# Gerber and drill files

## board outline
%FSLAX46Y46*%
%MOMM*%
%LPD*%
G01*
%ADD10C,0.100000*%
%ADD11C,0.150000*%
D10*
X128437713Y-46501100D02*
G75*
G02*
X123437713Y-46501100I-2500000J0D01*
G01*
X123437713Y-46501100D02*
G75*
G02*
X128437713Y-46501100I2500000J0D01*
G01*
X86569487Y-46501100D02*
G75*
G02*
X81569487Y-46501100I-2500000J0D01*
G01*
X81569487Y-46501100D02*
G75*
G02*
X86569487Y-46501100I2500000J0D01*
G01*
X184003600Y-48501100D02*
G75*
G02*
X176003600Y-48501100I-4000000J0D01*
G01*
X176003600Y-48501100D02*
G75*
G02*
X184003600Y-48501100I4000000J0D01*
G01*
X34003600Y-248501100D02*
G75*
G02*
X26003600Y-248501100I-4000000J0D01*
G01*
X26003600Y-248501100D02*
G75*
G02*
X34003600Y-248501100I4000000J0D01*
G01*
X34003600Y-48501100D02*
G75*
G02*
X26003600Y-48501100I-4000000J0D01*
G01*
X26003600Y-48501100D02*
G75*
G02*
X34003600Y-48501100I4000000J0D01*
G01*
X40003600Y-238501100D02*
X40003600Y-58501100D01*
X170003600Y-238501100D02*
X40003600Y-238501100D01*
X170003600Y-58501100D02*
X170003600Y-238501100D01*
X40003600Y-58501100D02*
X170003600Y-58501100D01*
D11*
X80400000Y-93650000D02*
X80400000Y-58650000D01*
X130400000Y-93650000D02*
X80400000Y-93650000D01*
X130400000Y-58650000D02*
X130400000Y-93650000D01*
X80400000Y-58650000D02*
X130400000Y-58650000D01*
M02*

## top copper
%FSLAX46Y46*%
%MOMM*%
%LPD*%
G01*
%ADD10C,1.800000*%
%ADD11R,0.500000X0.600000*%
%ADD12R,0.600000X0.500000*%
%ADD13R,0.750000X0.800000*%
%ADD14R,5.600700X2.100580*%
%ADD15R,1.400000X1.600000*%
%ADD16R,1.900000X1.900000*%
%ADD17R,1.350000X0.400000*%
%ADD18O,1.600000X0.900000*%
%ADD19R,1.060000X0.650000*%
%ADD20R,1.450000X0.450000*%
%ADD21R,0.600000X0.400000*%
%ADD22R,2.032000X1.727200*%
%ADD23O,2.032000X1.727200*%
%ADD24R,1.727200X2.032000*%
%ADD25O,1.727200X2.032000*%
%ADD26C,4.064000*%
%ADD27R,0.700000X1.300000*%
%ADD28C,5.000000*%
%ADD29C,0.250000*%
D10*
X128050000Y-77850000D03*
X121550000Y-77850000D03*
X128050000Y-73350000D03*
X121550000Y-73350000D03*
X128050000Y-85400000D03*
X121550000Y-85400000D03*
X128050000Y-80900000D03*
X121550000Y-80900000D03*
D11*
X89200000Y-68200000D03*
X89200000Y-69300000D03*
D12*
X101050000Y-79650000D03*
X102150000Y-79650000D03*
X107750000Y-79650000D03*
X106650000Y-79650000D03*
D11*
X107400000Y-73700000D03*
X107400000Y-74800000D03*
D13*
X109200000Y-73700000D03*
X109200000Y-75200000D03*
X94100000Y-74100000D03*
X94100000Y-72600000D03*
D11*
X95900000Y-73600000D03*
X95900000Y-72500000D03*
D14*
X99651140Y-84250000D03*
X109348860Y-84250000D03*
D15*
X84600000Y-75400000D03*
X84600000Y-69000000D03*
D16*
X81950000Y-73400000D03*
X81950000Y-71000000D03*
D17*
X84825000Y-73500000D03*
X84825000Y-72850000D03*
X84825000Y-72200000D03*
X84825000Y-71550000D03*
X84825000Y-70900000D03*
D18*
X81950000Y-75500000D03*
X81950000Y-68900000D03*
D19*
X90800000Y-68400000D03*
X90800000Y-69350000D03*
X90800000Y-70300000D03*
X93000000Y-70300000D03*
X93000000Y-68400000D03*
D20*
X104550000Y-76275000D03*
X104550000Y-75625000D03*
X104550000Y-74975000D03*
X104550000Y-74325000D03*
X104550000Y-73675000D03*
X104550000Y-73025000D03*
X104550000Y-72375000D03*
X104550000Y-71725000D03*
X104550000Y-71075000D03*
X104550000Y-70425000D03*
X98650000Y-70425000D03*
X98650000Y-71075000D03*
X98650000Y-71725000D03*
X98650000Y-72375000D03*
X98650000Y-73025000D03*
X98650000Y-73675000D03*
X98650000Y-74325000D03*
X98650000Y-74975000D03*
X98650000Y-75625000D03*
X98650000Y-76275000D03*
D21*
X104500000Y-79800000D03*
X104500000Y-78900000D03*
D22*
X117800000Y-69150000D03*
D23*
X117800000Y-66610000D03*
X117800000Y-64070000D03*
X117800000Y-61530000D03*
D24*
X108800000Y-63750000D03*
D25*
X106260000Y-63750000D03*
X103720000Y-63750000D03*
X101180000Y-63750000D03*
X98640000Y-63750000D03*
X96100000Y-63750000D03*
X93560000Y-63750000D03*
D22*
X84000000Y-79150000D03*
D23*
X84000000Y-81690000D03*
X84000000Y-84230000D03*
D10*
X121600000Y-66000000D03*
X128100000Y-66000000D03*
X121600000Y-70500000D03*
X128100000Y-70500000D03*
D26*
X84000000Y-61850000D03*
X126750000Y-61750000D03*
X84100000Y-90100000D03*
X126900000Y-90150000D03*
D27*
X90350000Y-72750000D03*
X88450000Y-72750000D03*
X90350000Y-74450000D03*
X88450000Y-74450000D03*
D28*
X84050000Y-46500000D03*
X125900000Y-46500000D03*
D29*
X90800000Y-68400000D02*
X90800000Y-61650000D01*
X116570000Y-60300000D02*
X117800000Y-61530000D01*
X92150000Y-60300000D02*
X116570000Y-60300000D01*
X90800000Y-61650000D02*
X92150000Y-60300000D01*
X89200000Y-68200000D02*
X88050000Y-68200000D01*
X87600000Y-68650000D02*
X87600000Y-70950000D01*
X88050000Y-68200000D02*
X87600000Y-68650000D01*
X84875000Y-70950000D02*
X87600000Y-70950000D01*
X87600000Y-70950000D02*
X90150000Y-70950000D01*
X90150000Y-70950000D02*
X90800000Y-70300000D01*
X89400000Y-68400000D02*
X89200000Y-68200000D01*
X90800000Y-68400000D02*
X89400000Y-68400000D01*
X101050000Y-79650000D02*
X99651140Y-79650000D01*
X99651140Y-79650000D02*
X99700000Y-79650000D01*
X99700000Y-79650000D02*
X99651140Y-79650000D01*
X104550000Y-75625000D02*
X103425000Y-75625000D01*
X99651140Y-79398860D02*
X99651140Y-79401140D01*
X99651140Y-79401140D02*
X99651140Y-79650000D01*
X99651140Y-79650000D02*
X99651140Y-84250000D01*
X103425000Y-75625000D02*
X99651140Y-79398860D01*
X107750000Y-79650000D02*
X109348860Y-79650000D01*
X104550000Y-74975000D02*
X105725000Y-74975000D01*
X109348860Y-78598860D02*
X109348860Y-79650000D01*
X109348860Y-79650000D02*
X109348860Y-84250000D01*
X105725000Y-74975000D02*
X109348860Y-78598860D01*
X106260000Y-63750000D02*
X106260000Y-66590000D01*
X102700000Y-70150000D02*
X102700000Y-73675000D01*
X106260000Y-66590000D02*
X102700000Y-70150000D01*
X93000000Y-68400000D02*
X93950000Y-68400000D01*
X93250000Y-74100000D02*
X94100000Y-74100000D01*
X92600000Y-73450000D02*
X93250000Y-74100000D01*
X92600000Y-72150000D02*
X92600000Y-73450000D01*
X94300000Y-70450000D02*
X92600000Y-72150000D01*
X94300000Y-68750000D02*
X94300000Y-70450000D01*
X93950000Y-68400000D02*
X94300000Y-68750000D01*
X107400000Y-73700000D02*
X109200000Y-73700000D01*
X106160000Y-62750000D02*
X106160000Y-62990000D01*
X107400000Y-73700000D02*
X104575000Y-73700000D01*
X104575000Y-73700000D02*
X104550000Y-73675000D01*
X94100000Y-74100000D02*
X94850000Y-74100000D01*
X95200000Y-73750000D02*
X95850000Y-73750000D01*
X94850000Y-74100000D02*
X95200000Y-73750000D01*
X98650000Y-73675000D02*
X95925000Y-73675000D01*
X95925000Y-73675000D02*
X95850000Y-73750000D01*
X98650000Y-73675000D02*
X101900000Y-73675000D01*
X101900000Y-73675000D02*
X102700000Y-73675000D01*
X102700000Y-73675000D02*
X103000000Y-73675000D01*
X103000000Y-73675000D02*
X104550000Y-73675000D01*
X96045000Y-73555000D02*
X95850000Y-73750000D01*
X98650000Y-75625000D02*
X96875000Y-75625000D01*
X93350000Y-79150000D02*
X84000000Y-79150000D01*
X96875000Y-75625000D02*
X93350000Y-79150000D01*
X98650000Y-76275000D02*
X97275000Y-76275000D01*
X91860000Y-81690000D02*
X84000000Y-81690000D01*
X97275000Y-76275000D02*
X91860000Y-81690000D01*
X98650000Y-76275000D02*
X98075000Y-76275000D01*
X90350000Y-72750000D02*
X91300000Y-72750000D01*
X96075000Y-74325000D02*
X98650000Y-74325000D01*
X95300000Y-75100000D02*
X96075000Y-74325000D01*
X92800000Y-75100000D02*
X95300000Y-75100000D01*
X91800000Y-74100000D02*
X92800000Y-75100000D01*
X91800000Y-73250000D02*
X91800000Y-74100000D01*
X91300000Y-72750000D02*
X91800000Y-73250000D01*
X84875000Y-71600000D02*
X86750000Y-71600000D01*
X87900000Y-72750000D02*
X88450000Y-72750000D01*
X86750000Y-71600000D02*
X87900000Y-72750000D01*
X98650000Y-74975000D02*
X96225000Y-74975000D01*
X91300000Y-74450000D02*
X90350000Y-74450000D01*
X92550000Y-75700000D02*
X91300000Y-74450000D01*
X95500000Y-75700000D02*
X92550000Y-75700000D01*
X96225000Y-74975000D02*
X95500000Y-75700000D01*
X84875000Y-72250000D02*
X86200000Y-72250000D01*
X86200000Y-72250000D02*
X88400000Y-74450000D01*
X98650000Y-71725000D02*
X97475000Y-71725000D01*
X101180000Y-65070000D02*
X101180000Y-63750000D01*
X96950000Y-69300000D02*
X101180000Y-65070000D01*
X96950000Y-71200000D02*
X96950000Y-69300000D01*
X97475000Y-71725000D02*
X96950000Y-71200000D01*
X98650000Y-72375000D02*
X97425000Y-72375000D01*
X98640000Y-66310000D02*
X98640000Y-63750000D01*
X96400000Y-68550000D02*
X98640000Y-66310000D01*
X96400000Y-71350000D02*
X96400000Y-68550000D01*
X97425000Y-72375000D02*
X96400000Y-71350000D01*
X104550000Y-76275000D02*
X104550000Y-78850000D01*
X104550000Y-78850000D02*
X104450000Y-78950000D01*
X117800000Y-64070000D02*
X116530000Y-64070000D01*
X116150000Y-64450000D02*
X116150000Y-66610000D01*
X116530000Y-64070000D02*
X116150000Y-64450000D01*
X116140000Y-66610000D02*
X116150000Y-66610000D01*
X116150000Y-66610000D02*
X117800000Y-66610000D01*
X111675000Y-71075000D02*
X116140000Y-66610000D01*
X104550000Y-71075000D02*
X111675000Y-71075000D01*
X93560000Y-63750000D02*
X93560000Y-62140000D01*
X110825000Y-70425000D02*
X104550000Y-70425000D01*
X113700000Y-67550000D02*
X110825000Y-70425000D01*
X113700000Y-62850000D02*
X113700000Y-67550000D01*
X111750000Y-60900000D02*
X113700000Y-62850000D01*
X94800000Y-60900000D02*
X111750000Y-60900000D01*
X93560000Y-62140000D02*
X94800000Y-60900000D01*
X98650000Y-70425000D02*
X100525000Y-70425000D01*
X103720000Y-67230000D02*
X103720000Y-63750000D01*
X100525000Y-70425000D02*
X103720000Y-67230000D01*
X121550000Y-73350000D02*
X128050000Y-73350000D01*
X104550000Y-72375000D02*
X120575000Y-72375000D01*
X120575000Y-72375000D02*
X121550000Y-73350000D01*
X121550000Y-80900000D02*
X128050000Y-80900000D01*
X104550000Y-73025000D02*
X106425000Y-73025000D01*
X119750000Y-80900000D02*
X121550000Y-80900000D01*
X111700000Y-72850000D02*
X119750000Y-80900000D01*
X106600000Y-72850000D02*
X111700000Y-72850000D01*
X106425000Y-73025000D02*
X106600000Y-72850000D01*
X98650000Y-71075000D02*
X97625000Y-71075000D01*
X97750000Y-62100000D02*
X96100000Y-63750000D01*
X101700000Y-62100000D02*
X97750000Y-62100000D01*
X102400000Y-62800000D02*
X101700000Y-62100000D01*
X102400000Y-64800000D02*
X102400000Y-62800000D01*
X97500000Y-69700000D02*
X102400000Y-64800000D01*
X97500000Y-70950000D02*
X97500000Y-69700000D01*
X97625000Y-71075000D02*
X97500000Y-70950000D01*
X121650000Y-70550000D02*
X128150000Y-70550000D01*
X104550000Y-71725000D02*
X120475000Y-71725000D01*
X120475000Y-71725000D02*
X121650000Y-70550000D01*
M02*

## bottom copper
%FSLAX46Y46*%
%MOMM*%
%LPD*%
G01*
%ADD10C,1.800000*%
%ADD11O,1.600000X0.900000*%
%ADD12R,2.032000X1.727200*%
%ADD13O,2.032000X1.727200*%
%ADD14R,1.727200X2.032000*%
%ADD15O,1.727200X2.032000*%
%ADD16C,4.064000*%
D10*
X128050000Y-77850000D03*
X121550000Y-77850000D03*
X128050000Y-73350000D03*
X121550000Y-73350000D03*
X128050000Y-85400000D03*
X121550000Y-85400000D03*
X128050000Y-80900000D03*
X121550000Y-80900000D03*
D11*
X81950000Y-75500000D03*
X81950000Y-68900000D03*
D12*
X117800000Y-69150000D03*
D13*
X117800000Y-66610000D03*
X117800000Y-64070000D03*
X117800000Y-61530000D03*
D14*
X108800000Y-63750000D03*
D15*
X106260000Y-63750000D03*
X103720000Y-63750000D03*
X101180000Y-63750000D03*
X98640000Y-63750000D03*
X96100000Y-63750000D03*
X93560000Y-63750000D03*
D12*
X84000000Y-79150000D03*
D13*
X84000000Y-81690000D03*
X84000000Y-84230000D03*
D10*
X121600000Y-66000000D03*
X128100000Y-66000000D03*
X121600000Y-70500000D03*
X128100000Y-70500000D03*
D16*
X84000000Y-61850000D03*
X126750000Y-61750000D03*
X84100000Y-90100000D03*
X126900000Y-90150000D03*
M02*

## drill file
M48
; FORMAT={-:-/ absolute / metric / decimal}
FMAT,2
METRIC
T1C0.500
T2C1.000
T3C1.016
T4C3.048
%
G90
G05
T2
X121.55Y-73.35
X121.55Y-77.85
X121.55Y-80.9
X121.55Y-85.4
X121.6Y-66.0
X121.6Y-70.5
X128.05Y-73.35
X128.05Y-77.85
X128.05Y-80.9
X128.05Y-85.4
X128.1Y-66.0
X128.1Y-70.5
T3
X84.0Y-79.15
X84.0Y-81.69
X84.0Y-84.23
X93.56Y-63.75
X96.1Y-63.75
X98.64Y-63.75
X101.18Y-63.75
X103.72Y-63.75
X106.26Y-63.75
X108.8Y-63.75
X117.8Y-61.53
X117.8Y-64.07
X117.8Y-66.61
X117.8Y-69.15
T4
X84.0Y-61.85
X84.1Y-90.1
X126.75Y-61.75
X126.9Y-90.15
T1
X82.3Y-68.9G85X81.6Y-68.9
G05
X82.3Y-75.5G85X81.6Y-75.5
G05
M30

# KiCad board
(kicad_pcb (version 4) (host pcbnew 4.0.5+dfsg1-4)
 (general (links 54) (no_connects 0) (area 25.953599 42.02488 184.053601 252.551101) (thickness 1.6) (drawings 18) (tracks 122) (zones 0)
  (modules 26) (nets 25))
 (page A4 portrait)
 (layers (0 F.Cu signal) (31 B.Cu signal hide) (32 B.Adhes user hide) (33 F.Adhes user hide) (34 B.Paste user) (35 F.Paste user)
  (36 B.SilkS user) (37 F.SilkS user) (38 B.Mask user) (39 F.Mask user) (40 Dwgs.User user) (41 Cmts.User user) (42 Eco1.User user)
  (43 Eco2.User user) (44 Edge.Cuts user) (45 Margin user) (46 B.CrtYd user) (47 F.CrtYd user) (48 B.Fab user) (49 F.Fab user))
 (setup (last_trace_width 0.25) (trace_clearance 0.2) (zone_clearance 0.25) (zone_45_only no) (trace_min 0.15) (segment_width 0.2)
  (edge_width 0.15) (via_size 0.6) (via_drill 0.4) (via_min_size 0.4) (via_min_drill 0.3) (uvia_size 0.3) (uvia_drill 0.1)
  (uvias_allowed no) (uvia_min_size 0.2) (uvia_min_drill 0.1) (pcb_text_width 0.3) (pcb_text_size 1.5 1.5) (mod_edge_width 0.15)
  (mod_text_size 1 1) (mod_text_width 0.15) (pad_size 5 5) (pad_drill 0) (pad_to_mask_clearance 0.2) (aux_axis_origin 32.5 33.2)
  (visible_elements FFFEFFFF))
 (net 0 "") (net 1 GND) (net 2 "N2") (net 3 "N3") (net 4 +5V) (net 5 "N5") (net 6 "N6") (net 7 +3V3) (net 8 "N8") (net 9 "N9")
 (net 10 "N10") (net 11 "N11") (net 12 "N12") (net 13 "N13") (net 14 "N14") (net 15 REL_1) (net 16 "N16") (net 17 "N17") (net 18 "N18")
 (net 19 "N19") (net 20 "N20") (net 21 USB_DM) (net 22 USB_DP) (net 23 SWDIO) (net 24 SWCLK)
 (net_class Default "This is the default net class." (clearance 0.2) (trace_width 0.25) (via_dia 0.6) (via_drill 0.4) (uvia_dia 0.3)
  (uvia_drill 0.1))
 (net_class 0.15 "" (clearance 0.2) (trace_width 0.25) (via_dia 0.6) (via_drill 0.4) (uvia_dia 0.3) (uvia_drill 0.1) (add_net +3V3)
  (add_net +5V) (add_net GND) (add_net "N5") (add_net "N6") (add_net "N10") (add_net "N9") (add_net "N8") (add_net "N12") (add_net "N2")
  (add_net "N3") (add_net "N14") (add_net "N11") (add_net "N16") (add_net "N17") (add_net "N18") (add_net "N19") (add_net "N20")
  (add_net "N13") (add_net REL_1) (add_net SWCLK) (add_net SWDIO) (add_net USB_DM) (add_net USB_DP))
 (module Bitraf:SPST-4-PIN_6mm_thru (layer B.Cu) (at 124.8 75.6 180)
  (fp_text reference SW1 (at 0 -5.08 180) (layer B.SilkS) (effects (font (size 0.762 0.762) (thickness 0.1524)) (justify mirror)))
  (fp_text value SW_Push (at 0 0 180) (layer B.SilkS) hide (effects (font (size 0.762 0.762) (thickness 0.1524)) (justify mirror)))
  (pad 1 thru_hole circle (at -3.25 -2.25 180) (size 1.8 1.8) (drill 1) (layers *.Cu *.Mask B.SilkS) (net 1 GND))
  (pad 1 thru_hole circle (at 3.25 -2.25 180) (size 1.8 1.8) (drill 1) (layers *.Cu *.Mask B.SilkS) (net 1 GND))
  (pad 2 thru_hole circle (at -3.25 2.25 180) (size 1.8 1.8) (drill 1) (layers *.Cu *.Mask B.SilkS) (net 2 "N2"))
  (pad 2 thru_hole circle (at 3.25 2.25 180) (size 1.8 1.8) (drill 1) (layers *.Cu *.Mask B.SilkS) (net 2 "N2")))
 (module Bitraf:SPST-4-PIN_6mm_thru (layer B.Cu) (at 124.8 83.15 180)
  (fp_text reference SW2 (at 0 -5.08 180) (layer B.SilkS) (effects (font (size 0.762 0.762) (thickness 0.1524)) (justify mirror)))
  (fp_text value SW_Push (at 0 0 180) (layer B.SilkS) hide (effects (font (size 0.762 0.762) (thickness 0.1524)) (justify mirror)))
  (pad 1 thru_hole circle (at -3.25 -2.25 180) (size 1.8 1.8) (drill 1) (layers *.Cu *.Mask B.SilkS) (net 1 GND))
  (pad 1 thru_hole circle (at 3.25 -2.25 180) (size 1.8 1.8) (drill 1) (layers *.Cu *.Mask B.SilkS) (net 1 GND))
  (pad 2 thru_hole circle (at -3.25 2.25 180) (size 1.8 1.8) (drill 1) (layers *.Cu *.Mask B.SilkS) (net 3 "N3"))
  (pad 2 thru_hole circle (at 3.25 2.25 180) (size 1.8 1.8) (drill 1) (layers *.Cu *.Mask B.SilkS) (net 3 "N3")))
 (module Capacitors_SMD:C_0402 (layer F.Cu) (at 89.2 68.75 270)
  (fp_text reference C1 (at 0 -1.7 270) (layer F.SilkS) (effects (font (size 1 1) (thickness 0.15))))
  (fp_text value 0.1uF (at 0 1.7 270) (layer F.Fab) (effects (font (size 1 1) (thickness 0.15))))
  (pad 1 smd rect (at -0.55 0 270) (size 0.6 0.5) (layers F.Cu F.Paste F.Mask) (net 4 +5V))
  (pad 2 smd rect (at 0.55 0 270) (size 0.6 0.5) (layers F.Cu F.Paste F.Mask) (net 1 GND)))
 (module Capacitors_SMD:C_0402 (layer F.Cu) (at 101.6 79.65)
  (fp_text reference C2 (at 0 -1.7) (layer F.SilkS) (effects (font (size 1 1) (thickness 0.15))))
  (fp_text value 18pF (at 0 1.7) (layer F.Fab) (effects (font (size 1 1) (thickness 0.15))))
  (pad 1 smd rect (at -0.55 0) (size 0.6 0.5) (layers F.Cu F.Paste F.Mask) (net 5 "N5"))
  (pad 2 smd rect (at 0.55 0) (size 0.6 0.5) (layers F.Cu F.Paste F.Mask) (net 1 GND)))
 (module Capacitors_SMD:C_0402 (layer F.Cu) (at 107.2 79.65 180)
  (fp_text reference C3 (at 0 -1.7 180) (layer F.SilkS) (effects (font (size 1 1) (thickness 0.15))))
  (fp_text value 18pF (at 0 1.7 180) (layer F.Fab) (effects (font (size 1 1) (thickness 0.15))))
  (pad 1 smd rect (at -0.55 0 180) (size 0.6 0.5) (layers F.Cu F.Paste F.Mask) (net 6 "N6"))
  (pad 2 smd rect (at 0.55 0 180) (size 0.6 0.5) (layers F.Cu F.Paste F.Mask) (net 1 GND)))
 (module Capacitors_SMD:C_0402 (layer F.Cu) (at 107.4 74.25 270)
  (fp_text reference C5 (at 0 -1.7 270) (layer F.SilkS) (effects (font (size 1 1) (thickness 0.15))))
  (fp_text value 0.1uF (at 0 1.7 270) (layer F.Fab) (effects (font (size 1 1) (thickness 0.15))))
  (pad 1 smd rect (at -0.55 0 270) (size 0.6 0.5) (layers F.Cu F.Paste F.Mask) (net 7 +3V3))
  (pad 2 smd rect (at 0.55 0 270) (size 0.6 0.5) (layers F.Cu F.Paste F.Mask) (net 1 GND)))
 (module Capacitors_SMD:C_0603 (layer F.Cu) (at 109.2 74.45 270)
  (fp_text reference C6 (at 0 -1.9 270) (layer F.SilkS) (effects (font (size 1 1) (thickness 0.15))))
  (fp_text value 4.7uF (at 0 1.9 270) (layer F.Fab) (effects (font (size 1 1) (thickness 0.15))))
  (pad 1 smd rect (at -0.75 0 270) (size 0.8 0.75) (layers F.Cu F.Paste F.Mask) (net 7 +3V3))
  (pad 2 smd rect (at 0.75 0 270) (size 0.8 0.75) (layers F.Cu F.Paste F.Mask) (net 1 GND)))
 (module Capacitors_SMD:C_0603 (layer F.Cu) (at 94.1 73.35 90)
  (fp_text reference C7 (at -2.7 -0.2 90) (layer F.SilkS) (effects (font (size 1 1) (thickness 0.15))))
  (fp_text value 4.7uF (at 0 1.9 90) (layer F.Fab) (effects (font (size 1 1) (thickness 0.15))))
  (pad 1 smd rect (at -0.75 0 90) (size 0.8 0.75) (layers F.Cu F.Paste F.Mask) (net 7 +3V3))
  (pad 2 smd rect (at 0.75 0 90) (size 0.8 0.75) (layers F.Cu F.Paste F.Mask) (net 1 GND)))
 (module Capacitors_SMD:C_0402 (layer F.Cu) (at 95.9 73.05 90)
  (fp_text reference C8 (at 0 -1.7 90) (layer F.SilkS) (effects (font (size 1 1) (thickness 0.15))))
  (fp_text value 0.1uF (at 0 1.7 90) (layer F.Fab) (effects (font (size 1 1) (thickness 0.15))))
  (pad 1 smd rect (at -0.55 0 90) (size 0.6 0.5) (layers F.Cu F.Paste F.Mask) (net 7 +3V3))
  (pad 2 smd rect (at 0.55 0 90) (size 0.6 0.5) (layers F.Cu F.Paste F.Mask) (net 1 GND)))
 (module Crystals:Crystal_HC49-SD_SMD (layer F.Cu) (at 104.5 84.25)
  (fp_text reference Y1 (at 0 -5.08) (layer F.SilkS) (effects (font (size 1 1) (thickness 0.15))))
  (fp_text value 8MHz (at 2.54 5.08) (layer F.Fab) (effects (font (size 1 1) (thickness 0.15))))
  (pad 1 smd rect (at -4.84886 0) (size 5.6007 2.10058) (layers F.Cu F.Paste F.Mask) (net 5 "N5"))
  (pad 2 smd rect (at 4.84886 0) (size 5.6007 2.10058) (layers F.Cu F.Paste F.Mask) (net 6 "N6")))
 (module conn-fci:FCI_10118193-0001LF (layer F.Cu) (at 81.95 72.2 270) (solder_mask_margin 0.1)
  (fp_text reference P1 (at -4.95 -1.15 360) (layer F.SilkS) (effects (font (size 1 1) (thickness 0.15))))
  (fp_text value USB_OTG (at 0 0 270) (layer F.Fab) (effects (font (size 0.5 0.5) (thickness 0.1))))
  (pad SH smd rect (at 3.2 -2.65 270) (size 1.6 1.4) (layers F.Cu F.Paste F.Mask))
  (pad SH smd rect (at -3.2 -2.65 270) (size 1.6 1.4) (layers F.Cu F.Paste F.Mask))
  (pad SH smd rect (at 1.2 0 270) (size 1.9 1.9) (layers F.Cu F.Paste F.Mask))
  (pad SH smd rect (at -1.2 0 270) (size 1.9 1.9) (layers F.Cu F.Paste F.Mask))
  (pad 5 smd rect (at 1.3 -2.875 270) (size 0.4 1.35) (layers F.Cu F.Paste F.Mask) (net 1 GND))
  (pad 4 smd rect (at 0.65 -2.875 270) (size 0.4 1.35) (layers F.Cu F.Paste F.Mask) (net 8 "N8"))
  (pad 3 smd rect (at 0 -2.875 270) (size 0.4 1.35) (layers F.Cu F.Paste F.Mask) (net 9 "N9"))
  (pad 2 smd rect (at -0.65 -2.875 270) (size 0.4 1.35) (layers F.Cu F.Paste F.Mask) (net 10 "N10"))
  (pad 1 smd rect (at -1.3 -2.875 270) (size 0.4 1.35) (layers F.Cu F.Paste F.Mask) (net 4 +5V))
  (pad SH thru_hole oval (at 3.3 0 270) (size 0.9 1.6) (drill oval 0.5 1.2) (layers *.Cu *.Mask))
  (pad SH thru_hole oval (at -3.3 0 270) (size 0.9 1.6) (drill oval 0.5 1.2) (layers *.Cu *.Mask)))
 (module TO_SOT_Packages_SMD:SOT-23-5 (layer F.Cu) (at 91.9 69.35)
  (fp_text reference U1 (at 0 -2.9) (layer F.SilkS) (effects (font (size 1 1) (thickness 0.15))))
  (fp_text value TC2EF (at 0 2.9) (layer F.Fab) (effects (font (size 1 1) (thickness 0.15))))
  (pad 1 smd rect (at -1.1 -0.95) (size 1.06 0.65) (layers F.Cu F.Paste F.Mask) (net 4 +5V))
  (pad 2 smd rect (at -1.1 0) (size 1.06 0.65) (layers F.Cu F.Paste F.Mask) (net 1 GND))
  (pad 3 smd rect (at -1.1 0.95) (size 1.06 0.65) (layers F.Cu F.Paste F.Mask) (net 4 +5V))
  (pad 4 smd rect (at 1.1 0.95) (size 1.06 0.65) (layers F.Cu F.Paste F.Mask) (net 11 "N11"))
  (pad 5 smd rect (at 1.1 -0.95) (size 1.06 0.65) (layers F.Cu F.Paste F.Mask) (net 7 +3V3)))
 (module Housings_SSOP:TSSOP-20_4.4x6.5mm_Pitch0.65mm (layer F.Cu) (at 101.6 73.35 180)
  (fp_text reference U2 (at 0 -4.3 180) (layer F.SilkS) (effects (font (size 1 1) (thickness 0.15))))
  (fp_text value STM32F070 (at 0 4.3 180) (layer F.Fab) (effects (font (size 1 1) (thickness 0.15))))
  (pad 1 smd rect (at -2.95 -2.925 180) (size 1.45 0.45) (layers F.Cu F.Paste F.Mask) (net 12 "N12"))
  (pad 2 smd rect (at -2.95 -2.275 180) (size 1.45 0.45) (layers F.Cu F.Paste F.Mask) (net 5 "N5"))
  (pad 3 smd rect (at -2.95 -1.625 180) (size 1.45 0.45) (layers F.Cu F.Paste F.Mask) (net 6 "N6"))
  (pad 4 smd rect (at -2.95 -0.975 180) (size 1.45 0.45) (layers F.Cu F.Paste F.Mask) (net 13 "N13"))
  (pad 5 smd rect (at -2.95 -0.325 180) (size 1.45 0.45) (layers F.Cu F.Paste F.Mask) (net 7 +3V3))
  (pad 6 smd rect (at -2.95 0.325 180) (size 1.45 0.45) (layers F.Cu F.Paste F.Mask) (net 3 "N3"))
  (pad 7 smd rect (at -2.95 0.975 180) (size 1.45 0.45) (layers F.Cu F.Paste F.Mask) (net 2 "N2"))
  (pad 8 smd rect (at -2.95 1.625 180) (size 1.45 0.45) (layers F.Cu F.Paste F.Mask) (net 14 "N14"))
  (pad 9 smd rect (at -2.95 2.275 180) (size 1.45 0.45) (layers F.Cu F.Paste F.Mask) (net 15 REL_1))
  (pad 10 smd rect (at -2.95 2.925 180) (size 1.45 0.45) (layers F.Cu F.Paste F.Mask) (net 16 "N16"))
  (pad 11 smd rect (at 2.95 2.925 180) (size 1.45 0.45) (layers F.Cu F.Paste F.Mask) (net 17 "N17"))
  (pad 12 smd rect (at 2.95 2.275 180) (size 1.45 0.45) (layers F.Cu F.Paste F.Mask) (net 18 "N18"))
  (pad 13 smd rect (at 2.95 1.625 180) (size 1.45 0.45) (layers F.Cu F.Paste F.Mask) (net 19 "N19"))
  (pad 14 smd rect (at 2.95 0.975 180) (size 1.45 0.45) (layers F.Cu F.Paste F.Mask) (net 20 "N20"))
  (pad 15 smd rect (at 2.95 0.325 180) (size 1.45 0.45) (layers F.Cu F.Paste F.Mask) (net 1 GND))
  (pad 16 smd rect (at 2.95 -0.325 180) (size 1.45 0.45) (layers F.Cu F.Paste F.Mask) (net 7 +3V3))
  (pad 17 smd rect (at 2.95 -0.975 180) (size 1.45 0.45) (layers F.Cu F.Paste F.Mask) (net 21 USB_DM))
  (pad 18 smd rect (at 2.95 -1.625 180) (size 1.45 0.45) (layers F.Cu F.Paste F.Mask) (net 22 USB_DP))
  (pad 19 smd rect (at 2.95 -2.275 180) (size 1.45 0.45) (layers F.Cu F.Paste F.Mask) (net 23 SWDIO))
  (pad 20 smd rect (at 2.95 -2.925 180) (size 1.45 0.45) (layers F.Cu F.Paste F.Mask) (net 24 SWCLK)))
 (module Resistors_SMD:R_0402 (layer F.Cu) (at 104.5 79.35 90)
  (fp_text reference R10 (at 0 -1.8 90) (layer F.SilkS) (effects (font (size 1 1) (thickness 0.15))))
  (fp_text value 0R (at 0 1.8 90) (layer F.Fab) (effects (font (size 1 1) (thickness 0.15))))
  (pad 1 smd rect (at -0.45 0 90) (size 0.4 0.6) (layers F.Cu F.Paste F.Mask) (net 1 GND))
  (pad 2 smd rect (at 0.45 0 90) (size 0.4 0.6) (layers F.Cu F.Paste F.Mask) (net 12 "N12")))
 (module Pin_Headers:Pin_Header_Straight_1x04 (layer F.Cu) (at 117.8 69.15 180)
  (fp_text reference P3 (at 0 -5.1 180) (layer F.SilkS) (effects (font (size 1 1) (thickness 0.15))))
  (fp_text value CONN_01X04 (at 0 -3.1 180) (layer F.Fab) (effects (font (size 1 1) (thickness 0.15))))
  (pad 1 thru_hole rect (at 0 0 180) (size 2.032 1.7272) (drill 1.016) (layers *.Cu *.Mask) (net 1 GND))
  (pad 2 thru_hole oval (at 0 2.54 180) (size 2.032 1.7272) (drill 1.016) (layers *.Cu *.Mask) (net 15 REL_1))
  (pad 3 thru_hole oval (at 0 5.08 180) (size 2.032 1.7272) (drill 1.016) (layers *.Cu *.Mask) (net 15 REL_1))
  (pad 4 thru_hole oval (at 0 7.62 180) (size 2.032 1.7272) (drill 1.016) (layers *.Cu *.Mask) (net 4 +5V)))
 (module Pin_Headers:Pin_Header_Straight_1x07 (layer F.Cu) (at 108.8 63.75 270)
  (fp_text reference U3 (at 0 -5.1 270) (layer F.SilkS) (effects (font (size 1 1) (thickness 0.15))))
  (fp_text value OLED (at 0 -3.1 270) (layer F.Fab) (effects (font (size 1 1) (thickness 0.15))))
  (pad 1 thru_hole rect (at 0 0 270) (size 2.032 1.7272) (drill 1.016) (layers *.Cu *.Mask) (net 1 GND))
  (pad 2 thru_hole oval (at 0 2.54 270) (size 2.032 1.7272) (drill 1.016) (layers *.Cu *.Mask) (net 7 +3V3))
  (pad 3 thru_hole oval (at 0 5.08 270) (size 2.032 1.7272) (drill 1.016) (layers *.Cu *.Mask) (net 17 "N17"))
  (pad 4 thru_hole oval (at 0 7.62 270) (size 2.032 1.7272) (drill 1.016) (layers *.Cu *.Mask) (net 19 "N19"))
  (pad 5 thru_hole oval (at 0 10.16 270) (size 2.032 1.7272) (drill 1.016) (layers *.Cu *.Mask) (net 20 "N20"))
  (pad 6 thru_hole oval (at 0 12.7 270) (size 2.032 1.7272) (drill 1.016) (layers *.Cu *.Mask) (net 18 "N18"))
  (pad 7 thru_hole oval (at 0 15.24 270) (size 2.032 1.7272) (drill 1.016) (layers *.Cu *.Mask) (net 16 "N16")))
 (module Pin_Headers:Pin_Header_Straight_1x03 (layer F.Cu) (at 84 79.15)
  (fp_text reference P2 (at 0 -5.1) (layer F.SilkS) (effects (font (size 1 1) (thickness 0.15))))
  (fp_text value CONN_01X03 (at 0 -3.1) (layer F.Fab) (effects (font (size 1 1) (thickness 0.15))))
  (pad 1 thru_hole rect (at 0 0) (size 2.032 1.7272) (drill 1.016) (layers *.Cu *.Mask) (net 23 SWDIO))
  (pad 2 thru_hole oval (at 0 2.54) (size 2.032 1.7272) (drill 1.016) (layers *.Cu *.Mask) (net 24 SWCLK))
  (pad 3 thru_hole oval (at 0 5.08) (size 2.032 1.7272) (drill 1.016) (layers *.Cu *.Mask) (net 1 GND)))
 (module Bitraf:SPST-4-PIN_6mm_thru (layer B.Cu) (at 124.85 68.25)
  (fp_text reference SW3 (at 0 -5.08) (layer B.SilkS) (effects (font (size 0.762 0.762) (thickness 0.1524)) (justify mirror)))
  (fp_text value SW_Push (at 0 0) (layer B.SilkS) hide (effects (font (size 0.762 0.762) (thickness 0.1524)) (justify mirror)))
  (pad 1 thru_hole circle (at -3.25 -2.25) (size 1.8 1.8) (drill 1) (layers *.Cu *.Mask B.SilkS) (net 1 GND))
  (pad 1 thru_hole circle (at 3.25 -2.25) (size 1.8 1.8) (drill 1) (layers *.Cu *.Mask B.SilkS) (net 1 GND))
  (pad 2 thru_hole circle (at -3.25 2.25) (size 1.8 1.8) (drill 1) (layers *.Cu *.Mask B.SilkS) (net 14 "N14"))
  (pad 2 thru_hole circle (at 3.25 2.25) (size 1.8 1.8) (drill 1) (layers *.Cu *.Mask B.SilkS) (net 14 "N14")))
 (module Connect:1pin (layer F.Cu) (at 84 61.85)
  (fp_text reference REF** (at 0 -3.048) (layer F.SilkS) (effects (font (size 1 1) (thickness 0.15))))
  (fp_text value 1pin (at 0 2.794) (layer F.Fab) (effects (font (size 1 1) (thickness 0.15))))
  (pad 1 thru_hole circle (at 0 0) (size 4.064 4.064) (drill 3.048) (layers *.Cu *.Mask)))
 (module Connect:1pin (layer F.Cu) (at 126.75 61.75)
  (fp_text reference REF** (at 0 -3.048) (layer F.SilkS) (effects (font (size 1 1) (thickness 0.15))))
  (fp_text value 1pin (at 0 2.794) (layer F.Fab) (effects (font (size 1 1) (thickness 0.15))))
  (pad 1 thru_hole circle (at 0 0) (size 4.064 4.064) (drill 3.048) (layers *.Cu *.Mask)))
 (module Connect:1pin (layer F.Cu) (at 84.1 90.1)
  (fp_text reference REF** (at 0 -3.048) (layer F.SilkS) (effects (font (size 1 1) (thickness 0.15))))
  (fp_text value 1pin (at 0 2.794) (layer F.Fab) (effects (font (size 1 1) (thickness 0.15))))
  (pad 1 thru_hole circle (at 0 0) (size 4.064 4.064) (drill 3.048) (layers *.Cu *.Mask)))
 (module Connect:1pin (layer F.Cu) (at 126.9 90.15)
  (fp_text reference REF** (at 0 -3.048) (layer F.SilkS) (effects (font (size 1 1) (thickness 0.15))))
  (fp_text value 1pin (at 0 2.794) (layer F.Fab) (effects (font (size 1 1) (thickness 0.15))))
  (pad 1 thru_hole circle (at 0 0) (size 4.064 4.064) (drill 3.048) (layers *.Cu *.Mask)))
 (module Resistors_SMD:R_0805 (layer F.Cu) (at 89.4 72.75 180)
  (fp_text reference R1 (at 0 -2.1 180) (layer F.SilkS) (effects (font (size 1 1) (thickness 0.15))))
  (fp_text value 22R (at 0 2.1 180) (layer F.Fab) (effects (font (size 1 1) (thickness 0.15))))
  (pad 1 smd rect (at -0.95 0 180) (size 0.7 1.3) (layers F.Cu F.Paste F.Mask) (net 21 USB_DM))
  (pad 2 smd rect (at 0.95 0 180) (size 0.7 1.3) (layers F.Cu F.Paste F.Mask) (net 10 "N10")))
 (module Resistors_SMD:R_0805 (layer F.Cu) (at 89.4 74.45 180)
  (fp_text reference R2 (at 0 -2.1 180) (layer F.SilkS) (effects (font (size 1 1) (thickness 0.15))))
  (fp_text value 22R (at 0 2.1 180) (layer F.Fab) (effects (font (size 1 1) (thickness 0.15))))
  (pad 1 smd rect (at -0.95 0 180) (size 0.7 1.3) (layers F.Cu F.Paste F.Mask) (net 22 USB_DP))
  (pad 2 smd rect (at 0.95 0 180) (size 0.7 1.3) (layers F.Cu F.Paste F.Mask) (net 9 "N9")))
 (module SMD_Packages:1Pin (layer F.Cu) (at 84.05 46.5)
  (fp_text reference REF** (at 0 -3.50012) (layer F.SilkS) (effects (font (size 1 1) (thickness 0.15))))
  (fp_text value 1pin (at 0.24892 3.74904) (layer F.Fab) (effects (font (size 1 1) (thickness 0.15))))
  (pad 1 smd circle (at 0 0) (size 5 5) (layers F.Cu F.Paste F.Mask)))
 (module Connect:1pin (layer F.Cu) (at 125.9 46.5)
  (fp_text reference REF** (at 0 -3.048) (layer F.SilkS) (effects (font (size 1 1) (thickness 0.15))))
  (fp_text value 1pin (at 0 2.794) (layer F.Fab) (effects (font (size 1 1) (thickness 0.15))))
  (pad 1 smd circle (at 0 0) (size 5 5) (layers F.Cu F.Paste F.Mask)))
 (gr_circle (center 125.937713 46.5011) (end 128.437713 46.5011) (layer Edge.Cuts) (width 0.1))
 (gr_circle (center 84.069487 46.5011) (end 86.569487 46.5011) (layer Edge.Cuts) (width 0.1))
 (gr_circle (center 180.0036 48.5011) (end 184.0036 48.5011) (layer Edge.Cuts) (width 0.1))
 (gr_circle (center 30.0036 248.5011) (end 34.0036 248.5011) (layer Edge.Cuts) (width 0.1))
 (gr_circle (center 30.0036 48.5011) (end 34.0036 48.5011) (layer Edge.Cuts) (width 0.1))
 (gr_line (start 40.0036 238.5011) (end 40.0036 58.5011) (layer Edge.Cuts) (width 0.1))
 (gr_line (start 170.0036 238.5011) (end 40.0036 238.5011) (layer Edge.Cuts) (width 0.1))
 (gr_line (start 170.0036 58.5011) (end 170.0036 238.5011) (layer Edge.Cuts) (width 0.1))
 (gr_line (start 40.0036 58.5011) (end 170.0036 58.5011) (layer Edge.Cuts) (width 0.1))
 (gr_line (start 80.4 93.65) (end 80.4 58.65) (angle 90) (layer Edge.Cuts) (width 0.15))
 (gr_line (start 130.4 93.65) (end 80.4 93.65) (angle 90) (layer Edge.Cuts) (width 0.15))
 (gr_line (start 130.4 58.65) (end 130.4 93.65) (angle 90) (layer Edge.Cuts) (width 0.15))
 (gr_line (start 80.4 58.65) (end 130.4 58.65) (angle 90) (layer Edge.Cuts) (width 0.15))
 (segment (start 90.8 68.4) (end 90.8 61.65) (width 0.25) (layer F.Cu) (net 4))
 (segment (start 116.57 60.3) (end 117.8 61.53) (width 0.25) (layer F.Cu) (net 4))
 (segment (start 92.15 60.3) (end 116.57 60.3) (width 0.25) (layer F.Cu) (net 4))
 (segment (start 90.8 61.65) (end 92.15 60.3) (width 0.25) (layer F.Cu) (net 4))
 (segment (start 89.2 68.2) (end 88.05 68.2) (width 0.25) (layer F.Cu) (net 4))
 (segment (start 87.6 68.65) (end 87.6 70.95) (width 0.25) (layer F.Cu) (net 4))
 (segment (start 88.05 68.2) (end 87.6 68.65) (width 0.25) (layer F.Cu) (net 4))
 (segment (start 84.875 70.95) (end 87.6 70.95) (width 0.25) (layer F.Cu) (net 4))
 (segment (start 87.6 70.95) (end 90.15 70.95) (width 0.25) (layer F.Cu) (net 4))
 (segment (start 90.15 70.95) (end 90.8 70.3) (width 0.25) (layer F.Cu) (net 4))
 (segment (start 89.4 68.4) (end 89.2 68.2) (width 0.25) (layer F.Cu) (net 4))
 (segment (start 90.8 68.4) (end 89.4 68.4) (width 0.25) (layer F.Cu) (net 4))
 (segment (start 101.05 79.65) (end 99.65114 79.65) (width 0.25) (layer F.Cu) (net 5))
 (segment (start 99.65114 79.65) (end 99.7 79.65) (width 0.25) (layer F.Cu) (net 5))
 (segment (start 99.7 79.65) (end 99.65114 79.65) (width 0.25) (layer F.Cu) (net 5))
 (segment (start 104.55 75.625) (end 103.425 75.625) (width 0.25) (layer F.Cu) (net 5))
 (segment (start 99.65114 79.39886) (end 99.65114 79.40114) (width 0.25) (layer F.Cu) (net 5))
 (segment (start 99.65114 79.40114) (end 99.65114 79.65) (width 0.25) (layer F.Cu) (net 5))
 (segment (start 99.65114 79.65) (end 99.65114 84.25) (width 0.25) (layer F.Cu) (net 5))
 (segment (start 103.425 75.625) (end 99.65114 79.39886) (width 0.25) (layer F.Cu) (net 5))
 (segment (start 107.75 79.65) (end 109.34886 79.65) (width 0.25) (layer F.Cu) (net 6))
 (segment (start 104.55 74.975) (end 105.725 74.975) (width 0.25) (layer F.Cu) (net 6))
 (segment (start 109.34886 78.59886) (end 109.34886 79.65) (width 0.25) (layer F.Cu) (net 6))
 (segment (start 109.34886 79.65) (end 109.34886 84.25) (width 0.25) (layer F.Cu) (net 6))
 (segment (start 105.725 74.975) (end 109.34886 78.59886) (width 0.25) (layer F.Cu) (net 6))
 (segment (start 106.26 63.75) (end 106.26 66.59) (width 0.25) (layer F.Cu) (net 7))
 (segment (start 102.7 70.15) (end 102.7 73.675) (width 0.25) (layer F.Cu) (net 7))
 (segment (start 106.26 66.59) (end 102.7 70.15) (width 0.25) (layer F.Cu) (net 7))
 (segment (start 93 68.4) (end 93.95 68.4) (width 0.25) (layer F.Cu) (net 7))
 (segment (start 93.25 74.1) (end 94.1 74.1) (width 0.25) (layer F.Cu) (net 7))
 (segment (start 92.6 73.45) (end 93.25 74.1) (width 0.25) (layer F.Cu) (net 7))
 (segment (start 92.6 72.15) (end 92.6 73.45) (width 0.25) (layer F.Cu) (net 7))
 (segment (start 94.3 70.45) (end 92.6 72.15) (width 0.25) (layer F.Cu) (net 7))
 (segment (start 94.3 68.75) (end 94.3 70.45) (width 0.25) (layer F.Cu) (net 7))
 (segment (start 93.95 68.4) (end 94.3 68.75) (width 0.25) (layer F.Cu) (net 7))
 (segment (start 107.4 73.7) (end 109.2 73.7) (width 0.25) (layer F.Cu) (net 7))
 (segment (start 106.16 62.75) (end 106.16 62.99) (width 0.25) (layer F.Cu) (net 7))
 (segment (start 107.4 73.7) (end 104.575 73.7) (width 0.25) (layer F.Cu) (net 7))
 (segment (start 104.575 73.7) (end 104.55 73.675) (width 0.25) (layer F.Cu) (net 7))
 (segment (start 94.1 74.1) (end 94.85 74.1) (width 0.25) (layer F.Cu) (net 7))
 (segment (start 95.2 73.75) (end 95.85 73.75) (width 0.25) (layer F.Cu) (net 7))
 (segment (start 94.85 74.1) (end 95.2 73.75) (width 0.25) (layer F.Cu) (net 7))
 (segment (start 98.65 73.675) (end 95.925 73.675) (width 0.25) (layer F.Cu) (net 7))
 (segment (start 95.925 73.675) (end 95.85 73.75) (width 0.25) (layer F.Cu) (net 7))
 (segment (start 98.65 73.675) (end 101.9 73.675) (width 0.25) (layer F.Cu) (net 7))
 (segment (start 101.9 73.675) (end 102.7 73.675) (width 0.25) (layer F.Cu) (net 7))
 (segment (start 102.7 73.675) (end 103 73.675) (width 0.25) (layer F.Cu) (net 7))
 (segment (start 103 73.675) (end 104.55 73.675) (width 0.25) (layer F.Cu) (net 7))
 (segment (start 96.045 73.555) (end 95.85 73.75) (width 0.25) (layer F.Cu) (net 7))
 (segment (start 98.65 75.625) (end 96.875 75.625) (width 0.25) (layer F.Cu) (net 23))
 (segment (start 93.35 79.15) (end 84 79.15) (width 0.25) (layer F.Cu) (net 23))
 (segment (start 96.875 75.625) (end 93.35 79.15) (width 0.25) (layer F.Cu) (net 23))
 (segment (start 98.65 76.275) (end 97.275 76.275) (width 0.25) (layer F.Cu) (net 24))
 (segment (start 91.86 81.69) (end 84 81.69) (width 0.25) (layer F.Cu) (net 24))
 (segment (start 97.275 76.275) (end 91.86 81.69) (width 0.25) (layer F.Cu) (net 24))
 (segment (start 98.65 76.275) (end 98.075 76.275) (width 0.25) (layer F.Cu) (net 24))
 (segment (start 90.35 72.75) (end 91.3 72.75) (width 0.25) (layer F.Cu) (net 21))
 (segment (start 96.075 74.325) (end 98.65 74.325) (width 0.25) (layer F.Cu) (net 21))
 (segment (start 95.3 75.1) (end 96.075 74.325) (width 0.25) (layer F.Cu) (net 21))
 (segment (start 92.8 75.1) (end 95.3 75.1) (width 0.25) (layer F.Cu) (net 21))
 (segment (start 91.8 74.1) (end 92.8 75.1) (width 0.25) (layer F.Cu) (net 21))
 (segment (start 91.8 73.25) (end 91.8 74.1) (width 0.25) (layer F.Cu) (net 21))
 (segment (start 91.3 72.75) (end 91.8 73.25) (width 0.25) (layer F.Cu) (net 21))
 (segment (start 84.875 71.6) (end 86.75 71.6) (width 0.25) (layer F.Cu) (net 10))
 (segment (start 87.9 72.75) (end 88.45 72.75) (width 0.25) (layer F.Cu) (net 10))
 (segment (start 86.75 71.6) (end 87.9 72.75) (width 0.25) (layer F.Cu) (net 10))
 (segment (start 98.65 74.975) (end 96.225 74.975) (width 0.25) (layer F.Cu) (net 22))
 (segment (start 91.3 74.45) (end 90.35 74.45) (width 0.25) (layer F.Cu) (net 22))
 (segment (start 92.55 75.7) (end 91.3 74.45) (width 0.25) (layer F.Cu) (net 22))
 (segment (start 95.5 75.7) (end 92.55 75.7) (width 0.25) (layer F.Cu) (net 22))
 (segment (start 96.225 74.975) (end 95.5 75.7) (width 0.25) (layer F.Cu) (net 22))
 (segment (start 84.875 72.25) (end 86.2 72.25) (width 0.25) (layer F.Cu) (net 9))
 (segment (start 86.2 72.25) (end 88.4 74.45) (width 0.25) (layer F.Cu) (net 9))
 (segment (start 98.65 71.725) (end 97.475 71.725) (width 0.25) (layer F.Cu) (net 19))
 (segment (start 101.18 65.07) (end 101.18 63.75) (width 0.25) (layer F.Cu) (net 19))
 (segment (start 96.95 69.3) (end 101.18 65.07) (width 0.25) (layer F.Cu) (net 19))
 (segment (start 96.95 71.2) (end 96.95 69.3) (width 0.25) (layer F.Cu) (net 19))
 (segment (start 97.475 71.725) (end 96.95 71.2) (width 0.25) (layer F.Cu) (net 19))
 (segment (start 98.65 72.375) (end 97.425 72.375) (width 0.25) (layer F.Cu) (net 20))
 (segment (start 98.64 66.31) (end 98.64 63.75) (width 0.25) (layer F.Cu) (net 20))
 (segment (start 96.4 68.55) (end 98.64 66.31) (width 0.25) (layer F.Cu) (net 20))
 (segment (start 96.4 71.35) (end 96.4 68.55) (width 0.25) (layer F.Cu) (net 20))
 (segment (start 97.425 72.375) (end 96.4 71.35) (width 0.25) (layer F.Cu) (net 20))
 (segment (start 104.55 76.275) (end 104.55 78.85) (width 0.25) (layer F.Cu) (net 12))
 (segment (start 104.55 78.85) (end 104.45 78.95) (width 0.25) (layer F.Cu) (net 12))
 (segment (start 117.8 64.07) (end 116.53 64.07) (width 0.25) (layer F.Cu) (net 15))
 (segment (start 116.15 64.45) (end 116.15 66.61) (width 0.25) (layer F.Cu) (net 15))
 (segment (start 116.53 64.07) (end 116.15 64.45) (width 0.25) (layer F.Cu) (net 15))
 (segment (start 116.14 66.61) (end 116.15 66.61) (width 0.25) (layer F.Cu) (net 15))
 (segment (start 116.15 66.61) (end 117.8 66.61) (width 0.25) (layer F.Cu) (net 15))
 (segment (start 111.675 71.075) (end 116.14 66.61) (width 0.25) (layer F.Cu) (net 15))
 (segment (start 104.55 71.075) (end 111.675 71.075) (width 0.25) (layer F.Cu) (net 15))
 (segment (start 93.56 63.75) (end 93.56 62.14) (width 0.25) (layer F.Cu) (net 16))
 (segment (start 110.825 70.425) (end 104.55 70.425) (width 0.25) (layer F.Cu) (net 16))
 (segment (start 113.7 67.55) (end 110.825 70.425) (width 0.25) (layer F.Cu) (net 16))
 (segment (start 113.7 62.85) (end 113.7 67.55) (width 0.25) (layer F.Cu) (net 16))
 (segment (start 111.75 60.9) (end 113.7 62.85) (width 0.25) (layer F.Cu) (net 16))
 (segment (start 94.8 60.9) (end 111.75 60.9) (width 0.25) (layer F.Cu) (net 16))
 (segment (start 93.56 62.14) (end 94.8 60.9) (width 0.25) (layer F.Cu) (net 16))
 (segment (start 98.65 70.425) (end 100.525 70.425) (width 0.25) (layer F.Cu) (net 17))
 (segment (start 103.72 67.23) (end 103.72 63.75) (width 0.25) (layer F.Cu) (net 17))
 (segment (start 100.525 70.425) (end 103.72 67.23) (width 0.25) (layer F.Cu) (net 17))
 (segment (start 121.55 73.35) (end 128.05 73.35) (width 0.25) (layer F.Cu) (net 2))
 (segment (start 104.55 72.375) (end 120.575 72.375) (width 0.25) (layer F.Cu) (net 2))
 (segment (start 120.575 72.375) (end 121.55 73.35) (width 0.25) (layer F.Cu) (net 2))
 (segment (start 121.55 80.9) (end 128.05 80.9) (width 0.25) (layer F.Cu) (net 3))
 (segment (start 104.55 73.025) (end 106.425 73.025) (width 0.25) (layer F.Cu) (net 3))
 (segment (start 119.75 80.9) (end 121.55 80.9) (width 0.25) (layer F.Cu) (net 3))
 (segment (start 111.7 72.85) (end 119.75 80.9) (width 0.25) (layer F.Cu) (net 3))
 (segment (start 106.6 72.85) (end 111.7 72.85) (width 0.25) (layer F.Cu) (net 3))
 (segment (start 106.425 73.025) (end 106.6 72.85) (width 0.25) (layer F.Cu) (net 3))
 (segment (start 98.65 71.075) (end 97.625 71.075) (width 0.25) (layer F.Cu) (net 18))
 (segment (start 97.75 62.1) (end 96.1 63.75) (width 0.25) (layer F.Cu) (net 18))
 (segment (start 101.7 62.1) (end 97.75 62.1) (width 0.25) (layer F.Cu) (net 18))
 (segment (start 102.4 62.8) (end 101.7 62.1) (width 0.25) (layer F.Cu) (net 18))
 (segment (start 102.4 64.8) (end 102.4 62.8) (width 0.25) (layer F.Cu) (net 18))
 (segment (start 97.5 69.7) (end 102.4 64.8) (width 0.25) (layer F.Cu) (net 18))
 (segment (start 97.5 70.95) (end 97.5 69.7) (width 0.25) (layer F.Cu) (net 18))
 (segment (start 97.625 71.075) (end 97.5 70.95) (width 0.25) (layer F.Cu) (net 18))
 (segment (start 121.65 70.55) (end 128.15 70.55) (width 0.25) (layer F.Cu) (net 14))
 (segment (start 104.55 71.725) (end 120.475 71.725) (width 0.25) (layer F.Cu) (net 14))
 (segment (start 120.475 71.725) (end 121.65 70.55) (width 0.25) (layer F.Cu) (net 14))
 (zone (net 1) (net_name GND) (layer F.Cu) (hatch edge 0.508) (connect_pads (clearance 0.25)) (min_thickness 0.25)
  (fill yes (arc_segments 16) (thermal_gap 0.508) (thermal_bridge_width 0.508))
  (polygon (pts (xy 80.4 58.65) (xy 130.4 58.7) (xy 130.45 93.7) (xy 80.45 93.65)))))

